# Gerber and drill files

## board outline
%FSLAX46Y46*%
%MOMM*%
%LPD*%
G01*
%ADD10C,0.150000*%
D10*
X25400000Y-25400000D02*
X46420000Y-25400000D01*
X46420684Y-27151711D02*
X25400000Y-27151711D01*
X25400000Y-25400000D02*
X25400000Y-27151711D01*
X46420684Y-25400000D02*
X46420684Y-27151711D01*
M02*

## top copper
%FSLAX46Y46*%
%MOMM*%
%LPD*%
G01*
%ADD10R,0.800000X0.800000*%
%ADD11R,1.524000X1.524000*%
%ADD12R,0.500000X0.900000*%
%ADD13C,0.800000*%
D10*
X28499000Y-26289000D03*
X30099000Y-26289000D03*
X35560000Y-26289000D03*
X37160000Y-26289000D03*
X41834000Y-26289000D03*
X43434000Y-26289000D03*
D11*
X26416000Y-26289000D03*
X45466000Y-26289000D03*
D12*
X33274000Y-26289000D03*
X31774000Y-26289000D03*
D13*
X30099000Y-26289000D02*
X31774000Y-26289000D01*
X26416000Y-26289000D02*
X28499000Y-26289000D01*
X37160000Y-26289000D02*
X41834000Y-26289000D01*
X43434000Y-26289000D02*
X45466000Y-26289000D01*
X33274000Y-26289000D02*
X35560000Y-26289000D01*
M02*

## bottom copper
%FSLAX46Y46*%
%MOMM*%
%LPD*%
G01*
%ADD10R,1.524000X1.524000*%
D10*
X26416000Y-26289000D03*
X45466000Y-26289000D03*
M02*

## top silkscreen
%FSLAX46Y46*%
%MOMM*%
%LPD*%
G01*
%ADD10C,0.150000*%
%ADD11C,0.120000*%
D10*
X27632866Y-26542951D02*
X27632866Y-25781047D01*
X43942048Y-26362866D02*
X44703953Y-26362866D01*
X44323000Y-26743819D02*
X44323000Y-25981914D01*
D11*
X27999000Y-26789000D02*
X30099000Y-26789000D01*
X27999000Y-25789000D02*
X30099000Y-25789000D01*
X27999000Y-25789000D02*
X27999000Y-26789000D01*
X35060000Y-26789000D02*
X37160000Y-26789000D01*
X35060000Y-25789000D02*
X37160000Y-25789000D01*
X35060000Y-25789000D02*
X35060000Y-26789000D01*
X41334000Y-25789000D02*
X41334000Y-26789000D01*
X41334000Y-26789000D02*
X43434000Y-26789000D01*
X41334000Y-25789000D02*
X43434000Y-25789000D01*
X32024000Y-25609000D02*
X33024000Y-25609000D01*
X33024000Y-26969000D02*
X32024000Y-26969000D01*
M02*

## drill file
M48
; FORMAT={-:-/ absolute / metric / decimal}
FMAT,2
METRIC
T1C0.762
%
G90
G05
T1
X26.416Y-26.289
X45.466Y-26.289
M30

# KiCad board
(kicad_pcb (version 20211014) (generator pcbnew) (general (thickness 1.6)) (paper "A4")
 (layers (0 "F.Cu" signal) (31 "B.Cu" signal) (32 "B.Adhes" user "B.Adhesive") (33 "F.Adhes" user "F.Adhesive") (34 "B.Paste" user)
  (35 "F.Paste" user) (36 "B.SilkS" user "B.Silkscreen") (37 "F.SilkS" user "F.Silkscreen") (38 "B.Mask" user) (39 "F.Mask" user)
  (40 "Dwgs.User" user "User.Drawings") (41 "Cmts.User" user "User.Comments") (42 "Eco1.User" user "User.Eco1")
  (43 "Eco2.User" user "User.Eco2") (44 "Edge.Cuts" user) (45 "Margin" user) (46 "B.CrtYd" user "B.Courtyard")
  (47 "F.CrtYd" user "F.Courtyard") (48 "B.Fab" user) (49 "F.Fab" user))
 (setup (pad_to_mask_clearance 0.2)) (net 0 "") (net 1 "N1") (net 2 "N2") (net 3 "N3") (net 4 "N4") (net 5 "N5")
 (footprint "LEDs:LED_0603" (layer "F.Cu") (at 29.299 26.289)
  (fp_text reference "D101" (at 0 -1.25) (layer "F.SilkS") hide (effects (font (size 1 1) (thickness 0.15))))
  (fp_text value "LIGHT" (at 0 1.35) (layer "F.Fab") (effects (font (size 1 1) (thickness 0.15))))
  (fp_line (start -1.3 0.5) (end 0.8 0.5) (layer "F.SilkS") (width 0.12))
  (fp_line (start -1.3 -0.5) (end 0.8 -0.5) (layer "F.SilkS") (width 0.12))
  (fp_line (start -1.3 -0.5) (end -1.3 0.5) (layer "F.SilkS") (width 0.12))
  (pad "1" smd rect locked (at -0.8 0 180) (size 0.8 0.8) (layers "F.Cu" "F.Paste" "F.Mask") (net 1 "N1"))
  (pad "2" smd rect locked (at 0.8 0 180) (size 0.8 0.8) (layers "F.Cu" "F.Paste" "F.Mask") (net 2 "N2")))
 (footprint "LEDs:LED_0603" (layer "F.Cu") (at 36.36 26.289)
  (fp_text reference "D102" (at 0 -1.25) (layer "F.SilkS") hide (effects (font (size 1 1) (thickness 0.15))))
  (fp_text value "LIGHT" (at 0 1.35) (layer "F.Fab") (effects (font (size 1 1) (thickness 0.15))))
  (fp_line (start -1.3 0.5) (end 0.8 0.5) (layer "F.SilkS") (width 0.12))
  (fp_line (start -1.3 -0.5) (end 0.8 -0.5) (layer "F.SilkS") (width 0.12))
  (fp_line (start -1.3 -0.5) (end -1.3 0.5) (layer "F.SilkS") (width 0.12))
  (pad "1" smd rect locked (at -0.8 0 180) (size 0.8 0.8) (layers "F.Cu" "F.Paste" "F.Mask") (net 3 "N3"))
  (pad "2" smd rect locked (at 0.8 0 180) (size 0.8 0.8) (layers "F.Cu" "F.Paste" "F.Mask") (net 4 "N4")))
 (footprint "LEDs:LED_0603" (layer "F.Cu") (at 42.634 26.289)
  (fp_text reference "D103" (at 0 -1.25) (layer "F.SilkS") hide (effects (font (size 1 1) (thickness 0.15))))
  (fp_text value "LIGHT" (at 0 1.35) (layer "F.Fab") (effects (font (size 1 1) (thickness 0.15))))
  (fp_line (start -1.3 -0.5) (end -1.3 0.5) (layer "F.SilkS") (width 0.12))
  (fp_line (start -1.3 0.5) (end 0.8 0.5) (layer "F.SilkS") (width 0.12))
  (fp_line (start -1.3 -0.5) (end 0.8 -0.5) (layer "F.SilkS") (width 0.12))
  (pad "1" smd rect locked (at -0.8 0 180) (size 0.8 0.8) (layers "F.Cu" "F.Paste" "F.Mask") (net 4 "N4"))
  (pad "2" smd rect locked (at 0.8 0 180) (size 0.8 0.8) (layers "F.Cu" "F.Paste" "F.Mask") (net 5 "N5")))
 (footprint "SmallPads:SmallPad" (layer "F.Cu") (at 26.416 26.289)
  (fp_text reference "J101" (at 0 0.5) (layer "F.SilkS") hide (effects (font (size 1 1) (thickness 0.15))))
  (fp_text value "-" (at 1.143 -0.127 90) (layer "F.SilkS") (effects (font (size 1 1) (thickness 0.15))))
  (pad "1" thru_hole rect locked (at 0 0) (size 1.524 1.524) (drill 0.762) (layers *.Cu *.Mask) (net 1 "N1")))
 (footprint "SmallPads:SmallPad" (layer "F.Cu") (at 45.466 26.289)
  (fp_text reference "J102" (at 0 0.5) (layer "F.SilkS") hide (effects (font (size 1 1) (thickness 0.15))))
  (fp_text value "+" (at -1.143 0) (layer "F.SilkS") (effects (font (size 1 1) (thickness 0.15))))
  (pad "1" thru_hole rect locked (at 0 0) (size 1.524 1.524) (drill 0.762) (layers *.Cu *.Mask) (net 5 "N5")))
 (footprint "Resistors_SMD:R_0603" (layer "F.Cu") (at 32.524 26.289 180)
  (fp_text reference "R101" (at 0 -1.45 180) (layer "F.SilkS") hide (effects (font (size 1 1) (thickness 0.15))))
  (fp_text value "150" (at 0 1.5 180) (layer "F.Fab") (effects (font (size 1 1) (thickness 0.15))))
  (fp_line (start 0.5 0.68) (end -0.5 0.68) (layer "F.SilkS") (width 0.12))
  (fp_line (start -0.5 -0.68) (end 0.5 -0.68) (layer "F.SilkS") (width 0.12))
  (pad "1" smd rect locked (at -0.75 0 180) (size 0.5 0.9) (layers "F.Cu" "F.Paste" "F.Mask") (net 3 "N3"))
  (pad "2" smd rect locked (at 0.75 0 180) (size 0.5 0.9) (layers "F.Cu" "F.Paste" "F.Mask") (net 2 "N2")))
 (gr_line (start 25.4 25.4) (end 46.42 25.4) (layer "Edge.Cuts") (width 0.15))
 (gr_line (start 46.420684 27.151711) (end 25.4 27.151711) (layer "Edge.Cuts") (width 0.15))
 (gr_line (start 25.4 25.4) (end 25.4 27.151711) (layer "Edge.Cuts") (width 0.15))
 (gr_line (start 46.420684 25.4) (end 46.420684 27.151711) (layer "Edge.Cuts") (width 0.15))
 (segment (start 30.099 26.289) (end 31.774 26.289) (width 0.8) (layer "F.Cu") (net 2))
 (segment (start 26.416 26.289) (end 28.499 26.289) (width 0.8) (layer "F.Cu") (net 1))
 (segment (start 37.16 26.289) (end 41.834 26.289) (width 0.8) (layer "F.Cu") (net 4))
 (segment (start 43.434 26.289) (end 45.466 26.289) (width 0.8) (layer "F.Cu") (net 5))
 (segment (start 33.274 26.289) (end 35.56 26.289) (width 0.8) (layer "F.Cu") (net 3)))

